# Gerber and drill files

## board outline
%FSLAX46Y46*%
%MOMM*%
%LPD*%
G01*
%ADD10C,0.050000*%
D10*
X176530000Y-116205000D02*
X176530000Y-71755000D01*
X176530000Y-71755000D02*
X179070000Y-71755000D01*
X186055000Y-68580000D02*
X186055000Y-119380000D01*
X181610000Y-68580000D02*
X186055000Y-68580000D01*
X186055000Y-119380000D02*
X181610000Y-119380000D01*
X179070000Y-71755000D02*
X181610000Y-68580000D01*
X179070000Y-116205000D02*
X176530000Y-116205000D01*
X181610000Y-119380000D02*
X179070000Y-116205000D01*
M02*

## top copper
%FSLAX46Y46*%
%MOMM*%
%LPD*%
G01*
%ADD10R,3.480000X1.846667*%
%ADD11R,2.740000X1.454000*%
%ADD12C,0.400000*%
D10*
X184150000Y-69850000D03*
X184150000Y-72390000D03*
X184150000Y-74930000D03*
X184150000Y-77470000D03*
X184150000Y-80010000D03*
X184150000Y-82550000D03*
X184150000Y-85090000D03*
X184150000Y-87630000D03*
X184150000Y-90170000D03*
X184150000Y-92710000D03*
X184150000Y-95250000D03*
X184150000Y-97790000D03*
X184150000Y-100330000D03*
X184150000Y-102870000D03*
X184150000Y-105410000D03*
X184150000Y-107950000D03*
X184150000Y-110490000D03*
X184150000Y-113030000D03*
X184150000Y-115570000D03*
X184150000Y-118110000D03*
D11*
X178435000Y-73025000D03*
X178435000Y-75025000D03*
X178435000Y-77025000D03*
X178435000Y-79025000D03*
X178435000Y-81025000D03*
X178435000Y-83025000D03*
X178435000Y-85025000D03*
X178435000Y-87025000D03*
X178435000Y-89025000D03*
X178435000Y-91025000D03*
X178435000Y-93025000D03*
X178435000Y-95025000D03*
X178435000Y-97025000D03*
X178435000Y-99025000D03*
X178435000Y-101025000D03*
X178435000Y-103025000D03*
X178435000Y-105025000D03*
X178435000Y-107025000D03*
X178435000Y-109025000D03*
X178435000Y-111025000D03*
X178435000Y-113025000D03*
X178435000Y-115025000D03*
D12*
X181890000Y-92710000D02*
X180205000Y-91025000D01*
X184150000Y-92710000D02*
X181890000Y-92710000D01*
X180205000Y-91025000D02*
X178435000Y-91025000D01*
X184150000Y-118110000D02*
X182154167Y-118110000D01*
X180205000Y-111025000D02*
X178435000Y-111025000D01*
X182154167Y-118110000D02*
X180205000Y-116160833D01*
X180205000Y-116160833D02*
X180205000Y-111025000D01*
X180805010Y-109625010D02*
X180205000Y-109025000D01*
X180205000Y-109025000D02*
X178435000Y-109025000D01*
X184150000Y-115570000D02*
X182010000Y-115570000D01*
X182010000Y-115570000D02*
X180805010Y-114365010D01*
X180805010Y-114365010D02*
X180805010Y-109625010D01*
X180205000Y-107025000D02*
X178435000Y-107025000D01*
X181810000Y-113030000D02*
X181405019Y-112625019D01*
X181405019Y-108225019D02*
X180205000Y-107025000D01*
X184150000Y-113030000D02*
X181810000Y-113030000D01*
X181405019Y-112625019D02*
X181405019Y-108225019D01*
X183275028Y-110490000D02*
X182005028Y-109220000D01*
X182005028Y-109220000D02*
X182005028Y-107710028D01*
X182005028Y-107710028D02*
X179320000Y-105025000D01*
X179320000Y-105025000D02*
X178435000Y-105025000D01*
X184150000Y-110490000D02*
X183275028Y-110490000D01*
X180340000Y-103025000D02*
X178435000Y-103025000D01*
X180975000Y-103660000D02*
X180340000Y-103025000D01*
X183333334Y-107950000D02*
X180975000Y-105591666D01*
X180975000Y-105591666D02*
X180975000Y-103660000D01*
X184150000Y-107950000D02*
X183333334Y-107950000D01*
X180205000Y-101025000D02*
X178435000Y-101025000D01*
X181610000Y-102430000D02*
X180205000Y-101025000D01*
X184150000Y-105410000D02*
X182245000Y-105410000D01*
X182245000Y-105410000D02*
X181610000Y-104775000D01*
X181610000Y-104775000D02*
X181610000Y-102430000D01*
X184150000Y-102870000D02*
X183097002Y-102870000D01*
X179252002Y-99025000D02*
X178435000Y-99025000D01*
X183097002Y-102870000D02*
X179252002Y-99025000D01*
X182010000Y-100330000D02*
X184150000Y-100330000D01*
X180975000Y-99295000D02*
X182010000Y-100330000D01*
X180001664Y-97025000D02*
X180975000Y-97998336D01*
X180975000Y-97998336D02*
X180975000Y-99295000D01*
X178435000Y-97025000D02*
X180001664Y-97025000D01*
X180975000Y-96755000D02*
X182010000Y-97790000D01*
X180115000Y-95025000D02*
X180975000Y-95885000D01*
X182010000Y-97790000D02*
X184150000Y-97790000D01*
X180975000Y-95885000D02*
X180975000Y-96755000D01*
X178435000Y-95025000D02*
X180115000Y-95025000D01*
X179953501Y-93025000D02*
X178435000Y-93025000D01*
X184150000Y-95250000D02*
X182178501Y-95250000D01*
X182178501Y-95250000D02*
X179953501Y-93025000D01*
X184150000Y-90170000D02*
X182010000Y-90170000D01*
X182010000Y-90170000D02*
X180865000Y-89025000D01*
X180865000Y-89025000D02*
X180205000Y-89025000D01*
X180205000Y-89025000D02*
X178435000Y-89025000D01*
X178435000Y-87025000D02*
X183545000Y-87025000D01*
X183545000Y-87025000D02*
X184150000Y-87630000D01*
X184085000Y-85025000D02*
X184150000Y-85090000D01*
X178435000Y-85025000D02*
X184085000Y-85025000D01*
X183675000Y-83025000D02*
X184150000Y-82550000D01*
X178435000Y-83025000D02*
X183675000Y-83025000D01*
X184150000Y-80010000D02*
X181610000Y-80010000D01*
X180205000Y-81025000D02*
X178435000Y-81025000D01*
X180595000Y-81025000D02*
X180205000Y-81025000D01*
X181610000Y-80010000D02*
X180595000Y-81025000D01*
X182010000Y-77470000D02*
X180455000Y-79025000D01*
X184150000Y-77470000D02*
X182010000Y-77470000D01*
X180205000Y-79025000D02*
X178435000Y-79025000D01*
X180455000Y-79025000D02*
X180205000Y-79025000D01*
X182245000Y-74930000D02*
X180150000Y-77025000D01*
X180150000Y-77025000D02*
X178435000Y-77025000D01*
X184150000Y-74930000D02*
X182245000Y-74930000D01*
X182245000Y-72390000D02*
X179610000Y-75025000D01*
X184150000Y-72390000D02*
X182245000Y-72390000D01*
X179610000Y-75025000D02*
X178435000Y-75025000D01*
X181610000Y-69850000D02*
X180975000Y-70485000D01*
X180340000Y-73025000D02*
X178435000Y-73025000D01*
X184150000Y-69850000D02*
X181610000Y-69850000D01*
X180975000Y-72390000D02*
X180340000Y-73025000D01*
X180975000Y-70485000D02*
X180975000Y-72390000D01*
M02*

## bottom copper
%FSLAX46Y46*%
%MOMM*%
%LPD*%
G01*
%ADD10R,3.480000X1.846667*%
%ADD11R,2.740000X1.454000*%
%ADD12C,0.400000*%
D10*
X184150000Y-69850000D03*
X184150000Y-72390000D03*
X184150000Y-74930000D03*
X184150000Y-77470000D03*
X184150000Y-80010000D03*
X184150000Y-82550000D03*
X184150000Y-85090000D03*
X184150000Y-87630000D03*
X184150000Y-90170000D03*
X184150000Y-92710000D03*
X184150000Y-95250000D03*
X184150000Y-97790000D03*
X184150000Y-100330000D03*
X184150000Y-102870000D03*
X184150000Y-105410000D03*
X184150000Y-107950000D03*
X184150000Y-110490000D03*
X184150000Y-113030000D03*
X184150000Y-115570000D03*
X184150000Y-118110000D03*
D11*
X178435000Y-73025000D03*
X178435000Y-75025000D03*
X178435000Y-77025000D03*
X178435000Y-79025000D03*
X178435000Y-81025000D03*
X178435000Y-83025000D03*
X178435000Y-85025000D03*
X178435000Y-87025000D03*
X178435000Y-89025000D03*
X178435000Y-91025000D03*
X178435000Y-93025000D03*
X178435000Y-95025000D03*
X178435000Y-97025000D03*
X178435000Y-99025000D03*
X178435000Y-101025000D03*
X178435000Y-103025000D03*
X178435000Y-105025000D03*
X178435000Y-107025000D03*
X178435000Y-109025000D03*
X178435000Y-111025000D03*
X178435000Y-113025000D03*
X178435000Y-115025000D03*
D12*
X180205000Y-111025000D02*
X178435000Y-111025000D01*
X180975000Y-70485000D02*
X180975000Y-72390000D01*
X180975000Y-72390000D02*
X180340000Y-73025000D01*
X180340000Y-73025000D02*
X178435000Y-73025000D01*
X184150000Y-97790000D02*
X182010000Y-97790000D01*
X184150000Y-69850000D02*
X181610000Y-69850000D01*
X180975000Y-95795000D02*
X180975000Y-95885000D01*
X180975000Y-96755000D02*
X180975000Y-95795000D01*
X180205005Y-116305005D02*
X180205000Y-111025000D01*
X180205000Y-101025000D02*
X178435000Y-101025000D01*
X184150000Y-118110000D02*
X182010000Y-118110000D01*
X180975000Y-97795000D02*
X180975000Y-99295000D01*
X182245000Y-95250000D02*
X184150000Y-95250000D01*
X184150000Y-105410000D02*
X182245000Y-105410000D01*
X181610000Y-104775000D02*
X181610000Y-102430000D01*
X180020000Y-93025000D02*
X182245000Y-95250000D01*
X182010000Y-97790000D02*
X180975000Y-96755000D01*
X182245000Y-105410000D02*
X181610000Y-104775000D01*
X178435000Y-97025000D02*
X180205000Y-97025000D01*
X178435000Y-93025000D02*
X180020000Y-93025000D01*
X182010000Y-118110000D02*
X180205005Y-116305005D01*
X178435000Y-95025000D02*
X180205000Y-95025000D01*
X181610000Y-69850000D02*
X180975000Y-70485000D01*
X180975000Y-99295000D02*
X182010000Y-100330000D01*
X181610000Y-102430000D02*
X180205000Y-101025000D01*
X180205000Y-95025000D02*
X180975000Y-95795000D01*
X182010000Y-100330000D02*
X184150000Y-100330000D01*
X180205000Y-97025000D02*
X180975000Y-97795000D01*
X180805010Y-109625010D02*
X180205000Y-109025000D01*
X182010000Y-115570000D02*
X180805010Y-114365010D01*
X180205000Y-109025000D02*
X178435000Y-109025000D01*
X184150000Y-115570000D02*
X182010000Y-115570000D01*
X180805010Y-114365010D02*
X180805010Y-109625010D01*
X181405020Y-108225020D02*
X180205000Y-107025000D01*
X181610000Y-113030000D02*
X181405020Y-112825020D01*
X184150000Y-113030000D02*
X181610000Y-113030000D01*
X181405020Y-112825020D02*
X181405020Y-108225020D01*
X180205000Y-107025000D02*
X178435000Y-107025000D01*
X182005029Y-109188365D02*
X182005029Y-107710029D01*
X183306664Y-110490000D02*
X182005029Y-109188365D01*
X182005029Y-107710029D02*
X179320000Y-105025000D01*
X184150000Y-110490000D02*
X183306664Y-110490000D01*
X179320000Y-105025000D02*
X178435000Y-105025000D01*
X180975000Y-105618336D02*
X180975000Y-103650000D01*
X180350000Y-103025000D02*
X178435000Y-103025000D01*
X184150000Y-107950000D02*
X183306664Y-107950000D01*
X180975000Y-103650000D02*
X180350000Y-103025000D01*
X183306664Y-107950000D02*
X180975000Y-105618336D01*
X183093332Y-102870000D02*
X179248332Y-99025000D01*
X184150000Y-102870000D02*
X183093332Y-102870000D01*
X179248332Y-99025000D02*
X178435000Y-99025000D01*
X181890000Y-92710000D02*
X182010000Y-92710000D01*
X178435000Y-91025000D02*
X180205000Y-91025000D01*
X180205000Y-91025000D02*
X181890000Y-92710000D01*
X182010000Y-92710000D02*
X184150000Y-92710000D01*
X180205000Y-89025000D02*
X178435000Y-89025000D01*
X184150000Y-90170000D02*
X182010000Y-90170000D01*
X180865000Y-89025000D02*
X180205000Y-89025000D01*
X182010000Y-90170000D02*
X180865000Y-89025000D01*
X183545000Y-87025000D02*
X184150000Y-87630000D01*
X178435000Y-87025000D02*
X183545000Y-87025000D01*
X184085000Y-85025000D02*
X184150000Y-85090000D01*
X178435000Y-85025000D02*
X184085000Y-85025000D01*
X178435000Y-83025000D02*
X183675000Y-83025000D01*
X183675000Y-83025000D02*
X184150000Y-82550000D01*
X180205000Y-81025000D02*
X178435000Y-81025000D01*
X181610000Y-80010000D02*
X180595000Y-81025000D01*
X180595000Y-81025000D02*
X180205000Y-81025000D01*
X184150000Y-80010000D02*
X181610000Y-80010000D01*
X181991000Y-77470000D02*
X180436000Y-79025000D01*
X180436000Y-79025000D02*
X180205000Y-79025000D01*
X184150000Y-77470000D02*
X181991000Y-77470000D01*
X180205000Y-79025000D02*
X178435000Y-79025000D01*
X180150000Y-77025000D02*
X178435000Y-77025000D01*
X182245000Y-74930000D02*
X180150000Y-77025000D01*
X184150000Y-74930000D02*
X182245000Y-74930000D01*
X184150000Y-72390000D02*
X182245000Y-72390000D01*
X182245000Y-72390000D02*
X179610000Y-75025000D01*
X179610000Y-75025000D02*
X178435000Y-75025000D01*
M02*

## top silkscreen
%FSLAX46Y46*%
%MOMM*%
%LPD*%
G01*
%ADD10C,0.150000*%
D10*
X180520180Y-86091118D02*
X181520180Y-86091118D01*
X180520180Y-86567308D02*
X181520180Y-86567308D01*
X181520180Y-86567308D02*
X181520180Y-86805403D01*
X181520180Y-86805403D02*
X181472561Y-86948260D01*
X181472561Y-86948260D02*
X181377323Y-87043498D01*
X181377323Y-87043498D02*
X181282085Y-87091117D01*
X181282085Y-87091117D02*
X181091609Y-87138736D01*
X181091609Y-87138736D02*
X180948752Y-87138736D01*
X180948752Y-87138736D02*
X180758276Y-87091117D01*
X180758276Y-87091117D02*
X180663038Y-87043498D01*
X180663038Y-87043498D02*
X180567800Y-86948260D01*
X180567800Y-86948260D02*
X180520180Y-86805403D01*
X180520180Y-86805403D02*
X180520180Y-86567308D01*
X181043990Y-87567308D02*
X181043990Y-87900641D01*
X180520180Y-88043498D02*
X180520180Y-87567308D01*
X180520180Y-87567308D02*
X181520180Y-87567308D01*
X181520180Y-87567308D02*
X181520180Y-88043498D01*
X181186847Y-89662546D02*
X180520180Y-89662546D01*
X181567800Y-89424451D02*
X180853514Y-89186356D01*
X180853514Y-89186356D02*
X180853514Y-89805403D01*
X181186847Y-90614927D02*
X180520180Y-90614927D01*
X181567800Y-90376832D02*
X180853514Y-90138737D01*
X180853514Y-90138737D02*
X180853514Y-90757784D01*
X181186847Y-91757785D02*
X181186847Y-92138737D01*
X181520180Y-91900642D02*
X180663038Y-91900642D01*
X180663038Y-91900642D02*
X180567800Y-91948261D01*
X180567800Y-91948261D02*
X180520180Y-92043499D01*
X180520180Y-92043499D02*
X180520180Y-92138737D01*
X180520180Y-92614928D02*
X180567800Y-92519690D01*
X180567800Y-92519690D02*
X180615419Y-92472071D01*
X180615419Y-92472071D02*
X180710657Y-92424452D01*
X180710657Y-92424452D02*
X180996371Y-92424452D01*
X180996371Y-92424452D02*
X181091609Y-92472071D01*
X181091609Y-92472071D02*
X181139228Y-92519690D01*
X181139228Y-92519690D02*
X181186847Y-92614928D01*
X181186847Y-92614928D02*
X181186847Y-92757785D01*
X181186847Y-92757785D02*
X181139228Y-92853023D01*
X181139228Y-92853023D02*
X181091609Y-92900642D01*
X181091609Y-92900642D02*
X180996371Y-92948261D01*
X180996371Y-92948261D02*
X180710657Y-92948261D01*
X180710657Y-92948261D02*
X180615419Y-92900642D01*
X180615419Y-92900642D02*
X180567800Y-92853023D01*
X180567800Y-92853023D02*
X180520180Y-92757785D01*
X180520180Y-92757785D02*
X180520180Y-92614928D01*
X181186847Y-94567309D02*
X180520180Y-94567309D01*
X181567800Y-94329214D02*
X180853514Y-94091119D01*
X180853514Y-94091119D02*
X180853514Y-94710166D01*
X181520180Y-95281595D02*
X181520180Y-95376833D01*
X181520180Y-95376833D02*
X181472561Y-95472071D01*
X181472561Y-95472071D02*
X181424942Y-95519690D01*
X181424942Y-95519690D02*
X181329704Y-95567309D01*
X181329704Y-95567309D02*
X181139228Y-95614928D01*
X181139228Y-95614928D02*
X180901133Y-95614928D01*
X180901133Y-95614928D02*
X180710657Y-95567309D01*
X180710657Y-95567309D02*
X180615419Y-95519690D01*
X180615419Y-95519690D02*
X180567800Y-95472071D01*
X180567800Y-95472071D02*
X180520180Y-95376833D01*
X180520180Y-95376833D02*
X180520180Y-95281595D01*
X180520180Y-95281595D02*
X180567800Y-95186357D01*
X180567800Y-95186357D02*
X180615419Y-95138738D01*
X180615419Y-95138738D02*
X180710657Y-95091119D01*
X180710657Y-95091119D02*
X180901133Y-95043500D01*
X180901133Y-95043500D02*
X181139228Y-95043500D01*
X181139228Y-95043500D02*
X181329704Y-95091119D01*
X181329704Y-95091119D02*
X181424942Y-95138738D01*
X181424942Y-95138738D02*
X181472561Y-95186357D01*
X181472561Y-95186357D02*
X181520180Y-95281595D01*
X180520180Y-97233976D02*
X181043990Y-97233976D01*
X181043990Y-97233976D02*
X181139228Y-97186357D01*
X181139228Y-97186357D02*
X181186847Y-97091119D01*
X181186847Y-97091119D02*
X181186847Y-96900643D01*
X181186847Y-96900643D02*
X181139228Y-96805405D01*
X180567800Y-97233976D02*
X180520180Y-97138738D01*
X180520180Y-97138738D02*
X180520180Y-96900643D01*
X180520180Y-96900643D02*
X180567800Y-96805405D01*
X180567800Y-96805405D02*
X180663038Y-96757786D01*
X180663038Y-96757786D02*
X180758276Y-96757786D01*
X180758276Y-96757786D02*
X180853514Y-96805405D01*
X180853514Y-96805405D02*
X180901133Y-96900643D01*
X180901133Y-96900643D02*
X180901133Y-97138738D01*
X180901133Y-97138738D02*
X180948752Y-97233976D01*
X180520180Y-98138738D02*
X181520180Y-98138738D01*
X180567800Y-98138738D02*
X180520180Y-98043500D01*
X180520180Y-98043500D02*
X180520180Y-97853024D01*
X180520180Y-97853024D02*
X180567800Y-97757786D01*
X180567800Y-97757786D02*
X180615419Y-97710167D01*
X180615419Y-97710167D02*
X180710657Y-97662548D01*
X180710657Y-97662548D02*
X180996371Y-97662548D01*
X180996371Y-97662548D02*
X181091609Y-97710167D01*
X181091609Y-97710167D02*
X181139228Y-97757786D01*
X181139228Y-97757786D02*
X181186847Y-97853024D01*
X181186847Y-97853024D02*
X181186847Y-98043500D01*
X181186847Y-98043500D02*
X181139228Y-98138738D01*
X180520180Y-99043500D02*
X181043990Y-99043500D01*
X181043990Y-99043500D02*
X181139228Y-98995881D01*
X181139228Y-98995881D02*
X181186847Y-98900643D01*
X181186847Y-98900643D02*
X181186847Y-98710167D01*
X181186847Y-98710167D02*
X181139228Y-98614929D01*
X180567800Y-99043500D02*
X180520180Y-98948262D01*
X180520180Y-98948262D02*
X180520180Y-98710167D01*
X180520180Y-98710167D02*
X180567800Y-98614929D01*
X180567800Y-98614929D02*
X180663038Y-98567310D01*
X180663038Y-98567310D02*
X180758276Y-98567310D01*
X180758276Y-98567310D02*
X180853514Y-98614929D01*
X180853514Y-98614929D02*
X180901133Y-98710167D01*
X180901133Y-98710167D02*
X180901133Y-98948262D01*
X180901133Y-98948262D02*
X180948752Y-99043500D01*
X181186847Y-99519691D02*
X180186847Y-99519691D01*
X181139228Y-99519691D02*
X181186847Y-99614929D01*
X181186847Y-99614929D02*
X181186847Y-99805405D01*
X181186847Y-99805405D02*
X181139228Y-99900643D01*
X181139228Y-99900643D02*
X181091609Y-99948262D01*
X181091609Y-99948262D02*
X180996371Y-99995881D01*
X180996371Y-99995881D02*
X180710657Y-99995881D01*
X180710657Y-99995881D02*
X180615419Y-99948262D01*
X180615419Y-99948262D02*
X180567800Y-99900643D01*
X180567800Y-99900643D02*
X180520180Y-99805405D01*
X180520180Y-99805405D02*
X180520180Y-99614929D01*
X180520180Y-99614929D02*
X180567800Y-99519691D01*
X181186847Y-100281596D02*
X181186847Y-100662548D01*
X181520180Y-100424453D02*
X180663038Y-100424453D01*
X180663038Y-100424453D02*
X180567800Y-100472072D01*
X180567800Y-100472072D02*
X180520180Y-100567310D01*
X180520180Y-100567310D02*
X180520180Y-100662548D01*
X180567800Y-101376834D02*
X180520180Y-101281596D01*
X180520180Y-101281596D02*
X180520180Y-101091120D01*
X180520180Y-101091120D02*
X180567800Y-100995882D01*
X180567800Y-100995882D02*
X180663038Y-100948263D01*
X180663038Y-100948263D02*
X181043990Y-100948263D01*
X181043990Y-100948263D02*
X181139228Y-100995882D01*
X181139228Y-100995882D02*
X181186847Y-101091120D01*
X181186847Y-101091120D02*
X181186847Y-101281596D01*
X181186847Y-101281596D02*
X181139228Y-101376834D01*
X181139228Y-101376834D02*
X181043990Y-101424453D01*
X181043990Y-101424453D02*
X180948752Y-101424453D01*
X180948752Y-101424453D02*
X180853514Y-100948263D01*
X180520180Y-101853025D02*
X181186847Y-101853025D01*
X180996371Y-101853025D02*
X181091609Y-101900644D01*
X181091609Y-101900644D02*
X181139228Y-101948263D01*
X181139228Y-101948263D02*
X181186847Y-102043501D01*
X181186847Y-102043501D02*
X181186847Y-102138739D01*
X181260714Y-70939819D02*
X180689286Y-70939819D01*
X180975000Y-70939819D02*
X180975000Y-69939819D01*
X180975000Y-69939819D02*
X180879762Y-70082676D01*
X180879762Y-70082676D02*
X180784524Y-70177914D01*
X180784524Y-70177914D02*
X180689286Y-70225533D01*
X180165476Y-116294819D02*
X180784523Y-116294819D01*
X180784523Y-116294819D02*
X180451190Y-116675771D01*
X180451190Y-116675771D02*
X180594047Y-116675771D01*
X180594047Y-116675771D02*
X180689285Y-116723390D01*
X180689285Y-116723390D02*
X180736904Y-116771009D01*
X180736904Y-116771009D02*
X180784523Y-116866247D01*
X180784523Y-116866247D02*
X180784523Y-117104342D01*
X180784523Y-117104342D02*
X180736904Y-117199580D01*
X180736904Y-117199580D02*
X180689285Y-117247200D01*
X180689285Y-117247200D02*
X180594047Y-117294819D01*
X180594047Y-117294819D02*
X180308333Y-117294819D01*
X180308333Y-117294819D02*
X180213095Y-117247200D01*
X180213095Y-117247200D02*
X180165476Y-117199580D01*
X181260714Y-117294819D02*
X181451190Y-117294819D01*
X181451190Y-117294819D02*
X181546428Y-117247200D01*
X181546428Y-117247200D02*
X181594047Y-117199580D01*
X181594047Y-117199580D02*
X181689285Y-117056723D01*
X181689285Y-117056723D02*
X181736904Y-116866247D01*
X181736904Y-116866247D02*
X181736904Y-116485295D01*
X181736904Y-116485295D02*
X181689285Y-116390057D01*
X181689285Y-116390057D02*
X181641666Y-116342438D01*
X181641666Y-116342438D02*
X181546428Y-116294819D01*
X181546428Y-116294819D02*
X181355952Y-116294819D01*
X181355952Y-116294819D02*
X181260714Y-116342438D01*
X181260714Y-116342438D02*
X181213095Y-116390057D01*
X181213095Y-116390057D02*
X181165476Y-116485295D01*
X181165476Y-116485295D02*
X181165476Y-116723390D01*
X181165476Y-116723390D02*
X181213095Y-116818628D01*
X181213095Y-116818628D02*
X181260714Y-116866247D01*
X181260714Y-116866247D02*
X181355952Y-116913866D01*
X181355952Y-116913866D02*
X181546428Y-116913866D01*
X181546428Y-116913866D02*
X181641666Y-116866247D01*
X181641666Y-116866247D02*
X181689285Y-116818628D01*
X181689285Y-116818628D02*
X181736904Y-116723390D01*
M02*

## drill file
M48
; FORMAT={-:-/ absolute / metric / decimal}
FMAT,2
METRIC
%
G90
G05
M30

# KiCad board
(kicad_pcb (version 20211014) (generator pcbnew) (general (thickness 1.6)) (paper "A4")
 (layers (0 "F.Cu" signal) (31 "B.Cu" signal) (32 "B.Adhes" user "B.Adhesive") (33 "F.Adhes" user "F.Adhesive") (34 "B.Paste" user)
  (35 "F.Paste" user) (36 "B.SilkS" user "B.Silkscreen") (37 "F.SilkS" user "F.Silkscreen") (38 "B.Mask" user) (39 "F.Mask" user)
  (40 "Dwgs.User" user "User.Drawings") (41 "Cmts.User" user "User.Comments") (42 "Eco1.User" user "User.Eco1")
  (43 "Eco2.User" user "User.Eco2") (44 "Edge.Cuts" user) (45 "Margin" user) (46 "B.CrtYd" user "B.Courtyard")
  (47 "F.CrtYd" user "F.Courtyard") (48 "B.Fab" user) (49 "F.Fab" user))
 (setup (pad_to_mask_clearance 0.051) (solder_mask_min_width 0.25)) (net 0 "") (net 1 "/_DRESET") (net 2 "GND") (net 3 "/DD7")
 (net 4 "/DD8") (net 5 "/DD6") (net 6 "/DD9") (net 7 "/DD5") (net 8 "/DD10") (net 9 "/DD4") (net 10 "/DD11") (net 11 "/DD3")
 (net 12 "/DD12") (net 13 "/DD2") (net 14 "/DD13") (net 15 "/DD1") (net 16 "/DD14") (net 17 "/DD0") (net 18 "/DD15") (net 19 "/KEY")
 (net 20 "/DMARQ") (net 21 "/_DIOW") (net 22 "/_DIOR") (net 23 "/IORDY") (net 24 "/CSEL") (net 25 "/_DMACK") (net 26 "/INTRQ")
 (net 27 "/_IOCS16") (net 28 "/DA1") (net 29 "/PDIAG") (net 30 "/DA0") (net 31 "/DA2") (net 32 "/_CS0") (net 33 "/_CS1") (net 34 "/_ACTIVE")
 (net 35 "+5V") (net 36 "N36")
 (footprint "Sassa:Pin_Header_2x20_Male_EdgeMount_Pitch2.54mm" (layer "B.Cu") (at 184.15 69.85 -90)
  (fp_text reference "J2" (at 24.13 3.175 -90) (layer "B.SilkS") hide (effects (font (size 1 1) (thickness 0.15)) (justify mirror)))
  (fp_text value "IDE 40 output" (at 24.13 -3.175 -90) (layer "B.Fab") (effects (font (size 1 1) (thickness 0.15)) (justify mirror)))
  (pad "1" smd rect locked (at 0 0 270) (size 1.846667 3.48) (layers "F.Cu" "F.Paste" "F.Mask") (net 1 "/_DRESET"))
  (pad "2" smd rect locked (at 0 0 270) (size 1.846667 3.48) (layers "B.Cu" "B.Paste" "B.Mask") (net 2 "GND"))
  (pad "3" smd rect locked (at 2.54 0 270) (size 1.846667 3.48) (layers "F.Cu" "F.Paste" "F.Mask") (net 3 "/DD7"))
  (pad "4" smd rect locked (at 2.54 0 270) (size 1.846667 3.48) (layers "B.Cu" "B.Paste" "B.Mask") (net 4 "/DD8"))
  (pad "5" smd rect locked (at 5.08 0 270) (size 1.846667 3.48) (layers "F.Cu" "F.Paste" "F.Mask") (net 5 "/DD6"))
  (pad "6" smd rect locked (at 5.08 0 270) (size 1.846667 3.48) (layers "B.Cu" "B.Paste" "B.Mask") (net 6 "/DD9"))
  (pad "7" smd rect locked (at 7.62 0 270) (size 1.846667 3.48) (layers "F.Cu" "F.Paste" "F.Mask") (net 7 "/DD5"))
  (pad "8" smd rect locked (at 7.62 0 270) (size 1.846667 3.48) (layers "B.Cu" "B.Paste" "B.Mask") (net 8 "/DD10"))
  (pad "9" smd rect locked (at 10.16 0 270) (size 1.846667 3.48) (layers "F.Cu" "F.Paste" "F.Mask") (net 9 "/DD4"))
  (pad "10" smd rect locked (at 10.16 0 270) (size 1.846667 3.48) (layers "B.Cu" "B.Paste" "B.Mask") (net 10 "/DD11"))
  (pad "11" smd rect locked (at 12.7 0 270) (size 1.846667 3.48) (layers "F.Cu" "F.Paste" "F.Mask") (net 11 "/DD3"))
  (pad "12" smd rect locked (at 12.7 0 270) (size 1.846667 3.48) (layers "B.Cu" "B.Paste" "B.Mask") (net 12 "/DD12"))
  (pad "13" smd rect locked (at 15.24 0 270) (size 1.846667 3.48) (layers "F.Cu" "F.Paste" "F.Mask") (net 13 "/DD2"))
  (pad "14" smd rect locked (at 15.24 0 270) (size 1.846667 3.48) (layers "B.Cu" "B.Paste" "B.Mask") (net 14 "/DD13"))
  (pad "15" smd rect locked (at 17.78 0 270) (size 1.846667 3.48) (layers "F.Cu" "F.Paste" "F.Mask") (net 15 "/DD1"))
  (pad "16" smd rect locked (at 17.78 0 270) (size 1.846667 3.48) (layers "B.Cu" "B.Paste" "B.Mask") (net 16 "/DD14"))
  (pad "17" smd rect locked (at 20.32 0 270) (size 1.846667 3.48) (layers "F.Cu" "F.Paste" "F.Mask") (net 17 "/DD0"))
  (pad "18" smd rect locked (at 20.32 0 270) (size 1.846667 3.48) (layers "B.Cu" "B.Paste" "B.Mask") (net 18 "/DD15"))
  (pad "19" smd rect locked (at 22.86 0 270) (size 1.846667 3.48) (layers "F.Cu" "F.Paste" "F.Mask") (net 2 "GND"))
  (pad "20" smd rect locked (at 22.86 0 270) (size 1.846667 3.48) (layers "B.Cu" "B.Paste" "B.Mask") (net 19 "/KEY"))
  (pad "21" smd rect locked (at 25.4 0 270) (size 1.846667 3.48) (layers "F.Cu" "F.Paste" "F.Mask") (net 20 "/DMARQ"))
  (pad "22" smd rect locked (at 25.4 0 270) (size 1.846667 3.48) (layers "B.Cu" "B.Paste" "B.Mask") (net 2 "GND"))
  (pad "23" smd rect locked (at 27.94 0 270) (size 1.846667 3.48) (layers "F.Cu" "F.Paste" "F.Mask") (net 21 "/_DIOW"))
  (pad "24" smd rect locked (at 27.94 0 270) (size 1.846667 3.48) (layers "B.Cu" "B.Paste" "B.Mask") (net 2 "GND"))
  (pad "25" smd rect locked (at 30.48 0 270) (size 1.846667 3.48) (layers "F.Cu" "F.Paste" "F.Mask") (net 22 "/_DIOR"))
  (pad "26" smd rect locked (at 30.48 0 270) (size 1.846667 3.48) (layers "B.Cu" "B.Paste" "B.Mask") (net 2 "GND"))
  (pad "27" smd rect locked (at 33.02 0 270) (size 1.846667 3.48) (layers "F.Cu" "F.Paste" "F.Mask") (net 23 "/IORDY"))
  (pad "28" smd rect locked (at 33.02 0 270) (size 1.846667 3.48) (layers "B.Cu" "B.Paste" "B.Mask") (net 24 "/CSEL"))
  (pad "29" smd rect locked (at 35.56 0 270) (size 1.846667 3.48) (layers "F.Cu" "F.Paste" "F.Mask") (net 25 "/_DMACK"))
  (pad "30" smd rect locked (at 35.56 0 270) (size 1.846667 3.48) (layers "B.Cu" "B.Paste" "B.Mask") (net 2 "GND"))
  (pad "31" smd rect locked (at 38.1 0 270) (size 1.846667 3.48) (layers "F.Cu" "F.Paste" "F.Mask") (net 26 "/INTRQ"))
  (pad "32" smd rect locked (at 38.1 0 270) (size 1.846667 3.48) (layers "B.Cu" "B.Paste" "B.Mask") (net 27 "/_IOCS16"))
  (pad "33" smd rect locked (at 40.64 0 270) (size 1.846667 3.48) (layers "F.Cu" "F.Paste" "F.Mask") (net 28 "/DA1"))
  (pad "34" smd rect locked (at 40.64 0 270) (size 1.846667 3.48) (layers "B.Cu" "B.Paste" "B.Mask") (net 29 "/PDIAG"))
  (pad "35" smd rect locked (at 43.18 0 270) (size 1.846667 3.48) (layers "F.Cu" "F.Paste" "F.Mask") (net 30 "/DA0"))
  (pad "36" smd rect locked (at 43.18 0 270) (size 1.846667 3.48) (layers "B.Cu" "B.Paste" "B.Mask") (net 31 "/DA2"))
  (pad "37" smd rect locked (at 45.72 0 270) (size 1.846667 3.48) (layers "F.Cu" "F.Paste" "F.Mask") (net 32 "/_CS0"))
  (pad "38" smd rect locked (at 45.72 0 270) (size 1.846667 3.48) (layers "B.Cu" "B.Paste" "B.Mask") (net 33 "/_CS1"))
  (pad "39" smd rect locked (at 48.26 0 270) (size 1.846667 3.48) (layers "F.Cu" "F.Paste" "F.Mask") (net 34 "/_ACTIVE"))
  (pad "40" smd rect locked (at 48.26 0 270) (size 1.846667 3.48) (layers "B.Cu" "B.Paste" "B.Mask") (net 2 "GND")))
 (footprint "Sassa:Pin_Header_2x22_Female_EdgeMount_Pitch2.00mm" (layer "B.Cu") (at 178.435 73.025 90)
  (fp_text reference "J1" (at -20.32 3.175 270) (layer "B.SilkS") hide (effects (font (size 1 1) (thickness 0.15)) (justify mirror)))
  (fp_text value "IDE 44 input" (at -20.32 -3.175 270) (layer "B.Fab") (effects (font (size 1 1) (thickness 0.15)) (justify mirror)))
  (pad "1" smd rect locked (at 0 0 90) (size 1.454 2.74) (layers "F.Cu" "F.Paste" "F.Mask") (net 1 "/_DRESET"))
  (pad "2" smd rect locked (at 0 0 90) (size 1.454 2.74) (layers "B.Cu" "B.Paste" "B.Mask") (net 2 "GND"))
  (pad "3" smd rect locked (at -2 0 90) (size 1.454 2.74) (layers "F.Cu" "F.Paste" "F.Mask") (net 3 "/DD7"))
  (pad "4" smd rect locked (at -2 0 90) (size 1.454 2.74) (layers "B.Cu" "B.Paste" "B.Mask") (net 4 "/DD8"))
  (pad "5" smd rect locked (at -4 0 90) (size 1.454 2.74) (layers "F.Cu" "F.Paste" "F.Mask") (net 5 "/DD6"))
  (pad "6" smd rect locked (at -4 0 90) (size 1.454 2.74) (layers "B.Cu" "B.Paste" "B.Mask") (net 6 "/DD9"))
  (pad "7" smd rect locked (at -6 0 90) (size 1.454 2.74) (layers "F.Cu" "F.Paste" "F.Mask") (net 7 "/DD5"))
  (pad "8" smd rect locked (at -6 0 90) (size 1.454 2.74) (layers "B.Cu" "B.Paste" "B.Mask") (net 8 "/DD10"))
  (pad "9" smd rect locked (at -8 0 90) (size 1.454 2.74) (layers "F.Cu" "F.Paste" "F.Mask") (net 9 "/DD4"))
  (pad "10" smd rect locked (at -8 0 90) (size 1.454 2.74) (layers "B.Cu" "B.Paste" "B.Mask") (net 10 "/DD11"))
  (pad "11" smd rect locked (at -10 0 90) (size 1.454 2.74) (layers "F.Cu" "F.Paste" "F.Mask") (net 11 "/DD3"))
  (pad "12" smd rect locked (at -10 0 90) (size 1.454 2.74) (layers "B.Cu" "B.Paste" "B.Mask") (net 12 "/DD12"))
  (pad "13" smd rect locked (at -12 0 90) (size 1.454 2.74) (layers "F.Cu" "F.Paste" "F.Mask") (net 13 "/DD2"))
  (pad "14" smd rect locked (at -12 0 90) (size 1.454 2.74) (layers "B.Cu" "B.Paste" "B.Mask") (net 14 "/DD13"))
  (pad "15" smd rect locked (at -14 0 90) (size 1.454 2.74) (layers "F.Cu" "F.Paste" "F.Mask") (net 15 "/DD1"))
  (pad "16" smd rect locked (at -14 0 90) (size 1.454 2.74) (layers "B.Cu" "B.Paste" "B.Mask") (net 16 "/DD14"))
  (pad "17" smd rect locked (at -16 0 90) (size 1.454 2.74) (layers "F.Cu" "F.Paste" "F.Mask") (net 17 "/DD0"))
  (pad "18" smd rect locked (at -16 0 90) (size 1.454 2.74) (layers "B.Cu" "B.Paste" "B.Mask") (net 18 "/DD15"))
  (pad "19" smd rect locked (at -18 0 90) (size 1.454 2.74) (layers "F.Cu" "F.Paste" "F.Mask") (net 2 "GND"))
  (pad "20" smd rect locked (at -18 0 90) (size 1.454 2.74) (layers "B.Cu" "B.Paste" "B.Mask") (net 19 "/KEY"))
  (pad "21" smd rect locked (at -20 0 90) (size 1.454 2.74) (layers "F.Cu" "F.Paste" "F.Mask") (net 20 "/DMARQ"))
  (pad "22" smd rect locked (at -20 0 90) (size 1.454 2.74) (layers "B.Cu" "B.Paste" "B.Mask") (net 2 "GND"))
  (pad "23" smd rect locked (at -22 0 90) (size 1.454 2.74) (layers "F.Cu" "F.Paste" "F.Mask") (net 21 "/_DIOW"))
  (pad "24" smd rect locked (at -22 0 90) (size 1.454 2.74) (layers "B.Cu" "B.Paste" "B.Mask") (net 2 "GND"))
  (pad "25" smd rect locked (at -24 0 90) (size 1.454 2.74) (layers "F.Cu" "F.Paste" "F.Mask") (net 22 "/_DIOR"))
  (pad "26" smd rect locked (at -24 0 90) (size 1.454 2.74) (layers "B.Cu" "B.Paste" "B.Mask") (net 2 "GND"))
  (pad "27" smd rect locked (at -26 0 90) (size 1.454 2.74) (layers "F.Cu" "F.Paste" "F.Mask") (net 23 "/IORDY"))
  (pad "28" smd rect locked (at -26 0 90) (size 1.454 2.74) (layers "B.Cu" "B.Paste" "B.Mask") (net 24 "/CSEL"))
  (pad "29" smd rect locked (at -28 0 90) (size 1.454 2.74) (layers "F.Cu" "F.Paste" "F.Mask") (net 25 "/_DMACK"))
  (pad "30" smd rect locked (at -28 0 90) (size 1.454 2.74) (layers "B.Cu" "B.Paste" "B.Mask") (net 2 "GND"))
  (pad "31" smd rect locked (at -30 0 90) (size 1.454 2.74) (layers "F.Cu" "F.Paste" "F.Mask") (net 26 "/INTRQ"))
  (pad "32" smd rect locked (at -30 0 90) (size 1.454 2.74) (layers "B.Cu" "B.Paste" "B.Mask") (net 27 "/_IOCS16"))
  (pad "33" smd rect locked (at -32 0 90) (size 1.454 2.74) (layers "F.Cu" "F.Paste" "F.Mask") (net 28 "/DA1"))
  (pad "34" smd rect locked (at -32 0 90) (size 1.454 2.74) (layers "B.Cu" "B.Paste" "B.Mask") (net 29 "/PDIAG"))
  (pad "35" smd rect locked (at -34 0 90) (size 1.454 2.74) (layers "F.Cu" "F.Paste" "F.Mask") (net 30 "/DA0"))
  (pad "36" smd rect locked (at -34 0 90) (size 1.454 2.74) (layers "B.Cu" "B.Paste" "B.Mask") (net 31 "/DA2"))
  (pad "37" smd rect locked (at -36 0 90) (size 1.454 2.74) (layers "F.Cu" "F.Paste" "F.Mask") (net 32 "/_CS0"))
  (pad "38" smd rect locked (at -36 0 90) (size 1.454 2.74) (layers "B.Cu" "B.Paste" "B.Mask") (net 33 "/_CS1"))
  (pad "39" smd rect locked (at -38 0 90) (size 1.454 2.74) (layers "F.Cu" "F.Paste" "F.Mask") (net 34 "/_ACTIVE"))
  (pad "40" smd rect locked (at -38 0 90) (size 1.454 2.74) (layers "B.Cu" "B.Paste" "B.Mask") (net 2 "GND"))
  (pad "41" smd rect locked (at -40 0 90) (size 1.454 2.74) (layers "F.Cu" "F.Paste" "F.Mask") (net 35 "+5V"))
  (pad "42" smd rect locked (at -40 0 90) (size 1.454 2.74) (layers "B.Cu" "B.Paste" "B.Mask") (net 35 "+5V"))
  (pad "43" smd rect locked (at -42 0 90) (size 1.454 2.74) (layers "F.Cu" "F.Paste" "F.Mask") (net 2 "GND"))
  (pad "44" smd rect locked (at -42 0 90) (size 1.454 2.74) (layers "B.Cu" "B.Paste" "B.Mask") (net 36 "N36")))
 (gr_line (start 176.53 116.205) (end 176.53 71.755) (layer "Edge.Cuts") (width 0.05))
 (gr_line (start 176.53 71.755) (end 179.07 71.755) (layer "Edge.Cuts") (width 0.05))
 (gr_line (start 186.055 68.58) (end 186.055 119.38) (layer "Edge.Cuts") (width 0.05))
 (gr_line (start 181.61 68.58) (end 186.055 68.58) (layer "Edge.Cuts") (width 0.05))
 (gr_line (start 186.055 119.38) (end 181.61 119.38) (layer "Edge.Cuts") (width 0.05))
 (gr_line (start 179.07 71.755) (end 181.61 68.58) (layer "Edge.Cuts") (width 0.05))
 (gr_line (start 179.07 116.205) (end 176.53 116.205) (layer "Edge.Cuts") (width 0.05))
 (gr_line (start 181.61 119.38) (end 179.07 116.205) (layer "Edge.Cuts") (width 0.05))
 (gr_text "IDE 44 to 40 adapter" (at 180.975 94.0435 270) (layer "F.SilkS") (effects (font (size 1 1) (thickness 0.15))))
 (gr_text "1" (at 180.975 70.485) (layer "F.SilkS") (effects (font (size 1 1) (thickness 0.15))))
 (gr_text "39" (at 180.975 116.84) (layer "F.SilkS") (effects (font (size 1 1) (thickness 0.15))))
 (segment (start 181.89 92.71) (end 180.205 91.025) (width 0.4) (layer "F.Cu") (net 2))
 (segment (start 184.15 92.71) (end 181.89 92.71) (width 0.4) (layer "F.Cu") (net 2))
 (segment (start 180.205 91.025) (end 178.435 91.025) (width 0.4) (layer "F.Cu") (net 2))
 (segment (start 180.205 111.025) (end 178.435 111.025) (width 0.4) (layer "B.Cu") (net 2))
 (segment (start 180.975 70.485) (end 180.975 72.39) (width 0.4) (layer "B.Cu") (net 2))
 (segment (start 180.975 72.39) (end 180.34 73.025) (width 0.4) (layer "B.Cu") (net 2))
 (segment (start 180.34 73.025) (end 178.435 73.025) (width 0.4) (layer "B.Cu") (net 2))
 (segment (start 184.15 97.79) (end 182.01 97.79) (width 0.4) (layer "B.Cu") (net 2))
 (segment (start 184.15 69.85) (end 181.61 69.85) (width 0.4) (layer "B.Cu") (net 2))
 (segment (start 180.975 95.795) (end 180.975 95.885) (width 0.4) (layer "B.Cu") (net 2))
 (segment (start 180.975 96.755) (end 180.975 95.795) (width 0.4) (layer "B.Cu") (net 2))
 (segment (start 180.205005 116.305005) (end 180.205 111.025) (width 0.4) (layer "B.Cu") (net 2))
 (segment (start 180.205 101.025) (end 178.435 101.025) (width 0.4) (layer "B.Cu") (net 2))
 (segment (start 184.15 118.11) (end 182.01 118.11) (width 0.4) (layer "B.Cu") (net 2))
 (segment (start 180.975 97.795) (end 180.975 99.295) (width 0.4) (layer "B.Cu") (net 2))
 (segment (start 182.245 95.25) (end 184.15 95.25) (width 0.4) (layer "B.Cu") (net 2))
 (segment (start 184.15 105.41) (end 182.245 105.41) (width 0.4) (layer "B.Cu") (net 2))
 (segment (start 181.61 104.775) (end 181.61 102.43) (width 0.4) (layer "B.Cu") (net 2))
 (segment (start 180.02 93.025) (end 182.245 95.25) (width 0.4) (layer "B.Cu") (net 2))
 (segment (start 182.01 97.79) (end 180.975 96.755) (width 0.4) (layer "B.Cu") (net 2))
 (segment (start 182.245 105.41) (end 181.61 104.775) (width 0.4) (layer "B.Cu") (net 2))
 (segment (start 178.435 97.025) (end 180.205 97.025) (width 0.4) (layer "B.Cu") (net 2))
 (segment (start 178.435 93.025) (end 180.02 93.025) (width 0.4) (layer "B.Cu") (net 2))
 (segment (start 182.01 118.11) (end 180.205005 116.305005) (width 0.4) (layer "B.Cu") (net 2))
 (segment (start 178.435 95.025) (end 180.205 95.025) (width 0.4) (layer "B.Cu") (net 2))
 (segment (start 181.61 69.85) (end 180.975 70.485) (width 0.4) (layer "B.Cu") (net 2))
 (segment (start 180.975 99.295) (end 182.01 100.33) (width 0.4) (layer "B.Cu") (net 2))
 (segment (start 181.61 102.43) (end 180.205 101.025) (width 0.4) (layer "B.Cu") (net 2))
 (segment (start 180.205 95.025) (end 180.975 95.795) (width 0.4) (layer "B.Cu") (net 2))
 (segment (start 182.01 100.33) (end 184.15 100.33) (width 0.4) (layer "B.Cu") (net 2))
 (segment (start 180.205 97.025) (end 180.975 97.795) (width 0.4) (layer "B.Cu") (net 2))
 (segment (start 180.80501 109.62501) (end 180.205 109.025) (width 0.4) (layer "B.Cu") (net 33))
 (segment (start 182.01 115.57) (end 180.80501 114.36501) (width 0.4) (layer "B.Cu") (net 33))
 (segment (start 180.205 109.025) (end 178.435 109.025) (width 0.4) (layer "B.Cu") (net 33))
 (segment (start 184.15 115.57) (end 182.01 115.57) (width 0.4) (layer "B.Cu") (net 33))
 (segment (start 180.80501 114.36501) (end 180.80501 109.62501) (width 0.4) (layer "B.Cu") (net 33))
 (segment (start 181.40502 108.22502) (end 180.205 107.025) (width 0.4) (layer "B.Cu") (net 31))
 (segment (start 181.61 113.03) (end 181.40502 112.82502) (width 0.4) (layer "B.Cu") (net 31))
 (segment (start 184.15 113.03) (end 181.61 113.03) (width 0.4) (layer "B.Cu") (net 31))
 (segment (start 181.40502 112.82502) (end 181.40502 108.22502) (width 0.4) (layer "B.Cu") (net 31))
 (segment (start 180.205 107.025) (end 178.435 107.025) (width 0.4) (layer "B.Cu") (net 31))
 (segment (start 182.005029 109.188365) (end 182.005029 107.710029) (width 0.4) (layer "B.Cu") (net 29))
 (segment (start 183.306664 110.49) (end 182.005029 109.188365) (width 0.4) (layer "B.Cu") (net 29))
 (segment (start 182.005029 107.710029) (end 179.32 105.025) (width 0.4) (layer "B.Cu") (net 29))
 (segment (start 184.15 110.49) (end 183.306664 110.49) (width 0.4) (layer "B.Cu") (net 29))
 (segment (start 179.32 105.025) (end 178.435 105.025) (width 0.4) (layer "B.Cu") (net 29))
 (segment (start 180.975 105.618336) (end 180.975 103.65) (width 0.4) (layer "B.Cu") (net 27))
 (segment (start 180.35 103.025) (end 178.435 103.025) (width 0.4) (layer "B.Cu") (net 27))
 (segment (start 184.15 107.95) (end 183.306664 107.95) (width 0.4) (layer "B.Cu") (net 27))
 (segment (start 180.975 103.65) (end 180.35 103.025) (width 0.4) (layer "B.Cu") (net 27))
 (segment (start 183.306664 107.95) (end 180.975 105.618336) (width 0.4) (layer "B.Cu") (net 27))
 (segment (start 183.093332 102.87) (end 179.248332 99.025) (width 0.4) (layer "B.Cu") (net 24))
 (segment (start 184.15 102.87) (end 183.093332 102.87) (width 0.4) (layer "B.Cu") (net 24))
 (segment (start 179.248332 99.025) (end 178.435 99.025) (width 0.4) (layer "B.Cu") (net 24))
 (segment (start 181.89 92.71) (end 182.01 92.71) (width 0.4) (layer "B.Cu") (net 19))
 (segment (start 178.435 91.025) (end 180.205 91.025) (width 0.4) (layer "B.Cu") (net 19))
 (segment (start 180.205 91.025) (end 181.89 92.71) (width 0.4) (layer "B.Cu") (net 19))
 (segment (start 182.01 92.71) (end 184.15 92.71) (width 0.4) (layer "B.Cu") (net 19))
 (segment (start 180.205 89.025) (end 178.435 89.025) (width 0.4) (layer "B.Cu") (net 18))
 (segment (start 184.15 90.17) (end 182.01 90.17) (width 0.4) (layer "B.Cu") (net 18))
 (segment (start 180.865 89.025) (end 180.205 89.025) (width 0.4) (layer "B.Cu") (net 18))
 (segment (start 182.01 90.17) (end 180.865 89.025) (width 0.4) (layer "B.Cu") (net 18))
 (segment (start 183.545 87.025) (end 184.15 87.63) (width 0.4) (layer "B.Cu") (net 16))
 (segment (start 178.435 87.025) (end 183.545 87.025) (width 0.4) (layer "B.Cu") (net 16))
 (segment (start 184.085 85.025) (end 184.15 85.09) (width 0.4) (layer "B.Cu") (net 14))
 (segment (start 178.435 85.025) (end 184.085 85.025) (width 0.4) (layer "B.Cu") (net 14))
 (segment (start 178.435 83.025) (end 183.675 83.025) (width 0.4) (layer "B.Cu") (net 12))
 (segment (start 183.675 83.025) (end 184.15 82.55) (width 0.4) (layer "B.Cu") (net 12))
 (segment (start 180.205 81.025) (end 178.435 81.025) (width 0.4) (layer "B.Cu") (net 10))
 (segment (start 181.61 80.01) (end 180.595 81.025) (width 0.4) (layer "B.Cu") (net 10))
 (segment (start 180.595 81.025) (end 180.205 81.025) (width 0.4) (layer "B.Cu") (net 10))
 (segment (start 184.15 80.01) (end 181.61 80.01) (width 0.4) (layer "B.Cu") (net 10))
 (segment (start 181.991 77.47) (end 180.436 79.025) (width 0.4) (layer "B.Cu") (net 8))
 (segment (start 180.436 79.025) (end 180.205 79.025) (width 0.4) (layer "B.Cu") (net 8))
 (segment (start 184.15 77.47) (end 181.991 77.47) (width 0.4) (layer "B.Cu") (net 8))
 (segment (start 180.205 79.025) (end 178.435 79.025) (width 0.4) (layer "B.Cu") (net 8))
 (segment (start 180.15 77.025) (end 178.435 77.025) (width 0.4) (layer "B.Cu") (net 6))
 (segment (start 182.245 74.93) (end 180.15 77.025) (width 0.4) (layer "B.Cu") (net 6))
 (segment (start 184.15 74.93) (end 182.245 74.93) (width 0.4) (layer "B.Cu") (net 6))
 (segment (start 184.15 72.39) (end 182.245 72.39) (width 0.4) (layer "B.Cu") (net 4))
 (segment (start 182.245 72.39) (end 179.61 75.025) (width 0.4) (layer "B.Cu") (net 4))
 (segment (start 179.61 75.025) (end 178.435 75.025) (width 0.4) (layer "B.Cu") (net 4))
 (segment (start 184.15 118.11) (end 182.154167 118.11) (width 0.4) (layer "F.Cu") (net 34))
 (segment (start 180.205 111.025) (end 178.435 111.025) (width 0.4) (layer "F.Cu") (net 34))
 (segment (start 182.154167 118.11) (end 180.205 116.160833) (width 0.4) (layer "F.Cu") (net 34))
 (segment (start 180.205 116.160833) (end 180.205 111.025) (width 0.4) (layer "F.Cu") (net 34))
 (segment (start 180.80501 109.62501) (end 180.205 109.025) (width 0.4) (layer "F.Cu") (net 32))
 (segment (start 180.205 109.025) (end 178.435 109.025) (width 0.4) (layer "F.Cu") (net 32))
 (segment (start 184.15 115.57) (end 182.01 115.57) (width 0.4) (layer "F.Cu") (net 32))
 (segment (start 182.01 115.57) (end 180.80501 114.36501) (width 0.4) (layer "F.Cu") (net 32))
 (segment (start 180.80501 114.36501) (end 180.80501 109.62501) (width 0.4) (layer "F.Cu") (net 32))
 (segment (start 180.205 107.025) (end 178.435 107.025) (width 0.4) (layer "F.Cu") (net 30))
 (segment (start 181.81 113.03) (end 181.405019 112.625019) (width 0.4) (layer "F.Cu") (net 30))
 (segment (start 181.405019 108.225019) (end 180.205 107.025) (width 0.4) (layer "F.Cu") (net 30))
 (segment (start 184.15 113.03) (end 181.81 113.03) (width 0.4) (layer "F.Cu") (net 30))
 (segment (start 181.405019 112.625019) (end 181.405019 108.225019) (width 0.4) (layer "F.Cu") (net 30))
 (segment (start 183.275028 110.49) (end 182.005028 109.22) (width 0.4) (layer "F.Cu") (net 28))
 (segment (start 182.005028 109.22) (end 182.005028 107.710028) (width 0.4) (layer "F.Cu") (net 28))
 (segment (start 182.005028 107.710028) (end 179.32 105.025) (width 0.4) (layer "F.Cu") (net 28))
 (segment (start 179.32 105.025) (end 178.435 105.025) (width 0.4) (layer "F.Cu") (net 28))
 (segment (start 184.15 110.49) (end 183.275028 110.49) (width 0.4) (layer "F.Cu") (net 28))
 (segment (start 180.34 103.025) (end 178.435 103.025) (width 0.4) (layer "F.Cu") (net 26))
 (segment (start 180.975 103.66) (end 180.34 103.025) (width 0.4) (layer "F.Cu") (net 26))
 (segment (start 183.333334 107.95) (end 180.975 105.591666) (width 0.4) (layer "F.Cu") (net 26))
 (segment (start 180.975 105.591666) (end 180.975 103.66) (width 0.4) (layer "F.Cu") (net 26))
 (segment (start 184.15 107.95) (end 183.333334 107.95) (width 0.4) (layer "F.Cu") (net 26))
 (segment (start 180.205 101.025) (end 178.435 101.025) (width 0.4) (layer "F.Cu") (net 25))
 (segment (start 181.61 102.43) (end 180.205 101.025) (width 0.4) (layer "F.Cu") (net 25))
 (segment (start 184.15 105.41) (end 182.245 105.41) (width 0.4) (layer "F.Cu") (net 25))
 (segment (start 182.245 105.41) (end 181.61 104.775) (width 0.4) (layer "F.Cu") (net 25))
 (segment (start 181.61 104.775) (end 181.61 102.43) (width 0.4) (layer "F.Cu") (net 25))
 (segment (start 184.15 102.87) (end 183.097002 102.87) (width 0.4) (layer "F.Cu") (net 23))
 (segment (start 179.252002 99.025) (end 178.435 99.025) (width 0.4) (layer "F.Cu") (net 23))
 (segment (start 183.097002 102.87) (end 179.252002 99.025) (width 0.4) (layer "F.Cu") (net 23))
 (segment (start 182.01 100.33) (end 184.15 100.33) (width 0.4) (layer "F.Cu") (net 22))
 (segment (start 180.975 99.295) (end 182.01 100.33) (width 0.4) (layer "F.Cu") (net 22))
 (segment (start 180.001664 97.025) (end 180.975 97.998336) (width 0.4) (layer "F.Cu") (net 22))
 (segment (start 180.975 97.998336) (end 180.975 99.295) (width 0.4) (layer "F.Cu") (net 22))
 (segment (start 178.435 97.025) (end 180.001664 97.025) (width 0.4) (layer "F.Cu") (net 22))
 (segment (start 180.975 96.755) (end 182.01 97.79) (width 0.4) (layer "F.Cu") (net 21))
 (segment (start 180.115 95.025) (end 180.975 95.885) (width 0.4) (layer "F.Cu") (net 21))
 (segment (start 182.01 97.79) (end 184.15 97.79) (width 0.4) (layer "F.Cu") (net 21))
 (segment (start 180.975 95.885) (end 180.975 96.755) (width 0.4) (layer "F.Cu") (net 21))
 (segment (start 178.435 95.025) (end 180.115 95.025) (width 0.4) (layer "F.Cu") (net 21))
 (segment (start 179.953501 93.025) (end 178.435 93.025) (width 0.4) (layer "F.Cu") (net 20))
 (segment (start 184.15 95.25) (end 182.178501 95.25) (width 0.4) (layer "F.Cu") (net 20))
 (segment (start 182.178501 95.25) (end 179.953501 93.025) (width 0.4) (layer "F.Cu") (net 20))
 (segment (start 184.15 90.17) (end 182.01 90.17) (width 0.4) (layer "F.Cu") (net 17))
 (segment (start 182.01 90.17) (end 180.865 89.025) (width 0.4) (layer "F.Cu") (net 17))
 (segment (start 180.865 89.025) (end 180.205 89.025) (width 0.4) (layer "F.Cu") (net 17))
 (segment (start 180.205 89.025) (end 178.435 89.025) (width 0.4) (layer "F.Cu") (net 17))
 (segment (start 178.435 87.025) (end 183.545 87.025) (width 0.4) (layer "F.Cu") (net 15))
 (segment (start 183.545 87.025) (end 184.15 87.63) (width 0.4) (layer "F.Cu") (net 15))
 (segment (start 184.085 85.025) (end 184.15 85.09) (width 0.4) (layer "F.Cu") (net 13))
 (segment (start 178.435 85.025) (end 184.085 85.025) (width 0.4) (layer "F.Cu") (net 13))
 (segment (start 183.675 83.025) (end 184.15 82.55) (width 0.4) (layer "F.Cu") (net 11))
 (segment (start 178.435 83.025) (end 183.675 83.025) (width 0.4) (layer "F.Cu") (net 11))
 (segment (start 184.15 80.01) (end 181.61 80.01) (width 0.4) (layer "F.Cu") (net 9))
 (segment (start 180.205 81.025) (end 178.435 81.025) (width 0.4) (layer "F.Cu") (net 9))
 (segment (start 180.595 81.025) (end 180.205 81.025) (width 0.4) (layer "F.Cu") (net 9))
 (segment (start 181.61 80.01) (end 180.595 81.025) (width 0.4) (layer "F.Cu") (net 9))
 (segment (start 182.01 77.47) (end 180.455 79.025) (width 0.4) (layer "F.Cu") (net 7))
 (segment (start 184.15 77.47) (end 182.01 77.47) (width 0.4) (layer "F.Cu") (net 7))
 (segment (start 180.205 79.025) (end 178.435 79.025) (width 0.4) (layer "F.Cu") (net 7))
 (segment (start 180.455 79.025) (end 180.205 79.025) (width 0.4) (layer "F.Cu") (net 7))
 (segment (start 182.245 74.93) (end 180.15 77.025) (width 0.4) (layer "F.Cu") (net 5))
 (segment (start 180.15 77.025) (end 178.435 77.025) (width 0.4) (layer "F.Cu") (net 5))
 (segment (start 184.15 74.93) (end 182.245 74.93) (width 0.4) (layer "F.Cu") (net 5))
 (segment (start 182.245 72.39) (end 179.61 75.025) (width 0.4) (layer "F.Cu") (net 3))
 (segment (start 184.15 72.39) (end 182.245 72.39) (width 0.4) (layer "F.Cu") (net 3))
 (segment (start 179.61 75.025) (end 178.435 75.025) (width 0.4) (layer "F.Cu") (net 3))
 (segment (start 181.61 69.85) (end 180.975 70.485) (width 0.4) (layer "F.Cu") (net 1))
 (segment (start 180.34 73.025) (end 178.435 73.025) (width 0.4) (layer "F.Cu") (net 1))
 (segment (start 184.15 69.85) (end 181.61 69.85) (width 0.4) (layer "F.Cu") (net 1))
 (segment (start 180.975 72.39) (end 180.34 73.025) (width 0.4) (layer "F.Cu") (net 1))
 (segment (start 180.975 70.485) (end 180.975 72.39) (width 0.4) (layer "F.Cu") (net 1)))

